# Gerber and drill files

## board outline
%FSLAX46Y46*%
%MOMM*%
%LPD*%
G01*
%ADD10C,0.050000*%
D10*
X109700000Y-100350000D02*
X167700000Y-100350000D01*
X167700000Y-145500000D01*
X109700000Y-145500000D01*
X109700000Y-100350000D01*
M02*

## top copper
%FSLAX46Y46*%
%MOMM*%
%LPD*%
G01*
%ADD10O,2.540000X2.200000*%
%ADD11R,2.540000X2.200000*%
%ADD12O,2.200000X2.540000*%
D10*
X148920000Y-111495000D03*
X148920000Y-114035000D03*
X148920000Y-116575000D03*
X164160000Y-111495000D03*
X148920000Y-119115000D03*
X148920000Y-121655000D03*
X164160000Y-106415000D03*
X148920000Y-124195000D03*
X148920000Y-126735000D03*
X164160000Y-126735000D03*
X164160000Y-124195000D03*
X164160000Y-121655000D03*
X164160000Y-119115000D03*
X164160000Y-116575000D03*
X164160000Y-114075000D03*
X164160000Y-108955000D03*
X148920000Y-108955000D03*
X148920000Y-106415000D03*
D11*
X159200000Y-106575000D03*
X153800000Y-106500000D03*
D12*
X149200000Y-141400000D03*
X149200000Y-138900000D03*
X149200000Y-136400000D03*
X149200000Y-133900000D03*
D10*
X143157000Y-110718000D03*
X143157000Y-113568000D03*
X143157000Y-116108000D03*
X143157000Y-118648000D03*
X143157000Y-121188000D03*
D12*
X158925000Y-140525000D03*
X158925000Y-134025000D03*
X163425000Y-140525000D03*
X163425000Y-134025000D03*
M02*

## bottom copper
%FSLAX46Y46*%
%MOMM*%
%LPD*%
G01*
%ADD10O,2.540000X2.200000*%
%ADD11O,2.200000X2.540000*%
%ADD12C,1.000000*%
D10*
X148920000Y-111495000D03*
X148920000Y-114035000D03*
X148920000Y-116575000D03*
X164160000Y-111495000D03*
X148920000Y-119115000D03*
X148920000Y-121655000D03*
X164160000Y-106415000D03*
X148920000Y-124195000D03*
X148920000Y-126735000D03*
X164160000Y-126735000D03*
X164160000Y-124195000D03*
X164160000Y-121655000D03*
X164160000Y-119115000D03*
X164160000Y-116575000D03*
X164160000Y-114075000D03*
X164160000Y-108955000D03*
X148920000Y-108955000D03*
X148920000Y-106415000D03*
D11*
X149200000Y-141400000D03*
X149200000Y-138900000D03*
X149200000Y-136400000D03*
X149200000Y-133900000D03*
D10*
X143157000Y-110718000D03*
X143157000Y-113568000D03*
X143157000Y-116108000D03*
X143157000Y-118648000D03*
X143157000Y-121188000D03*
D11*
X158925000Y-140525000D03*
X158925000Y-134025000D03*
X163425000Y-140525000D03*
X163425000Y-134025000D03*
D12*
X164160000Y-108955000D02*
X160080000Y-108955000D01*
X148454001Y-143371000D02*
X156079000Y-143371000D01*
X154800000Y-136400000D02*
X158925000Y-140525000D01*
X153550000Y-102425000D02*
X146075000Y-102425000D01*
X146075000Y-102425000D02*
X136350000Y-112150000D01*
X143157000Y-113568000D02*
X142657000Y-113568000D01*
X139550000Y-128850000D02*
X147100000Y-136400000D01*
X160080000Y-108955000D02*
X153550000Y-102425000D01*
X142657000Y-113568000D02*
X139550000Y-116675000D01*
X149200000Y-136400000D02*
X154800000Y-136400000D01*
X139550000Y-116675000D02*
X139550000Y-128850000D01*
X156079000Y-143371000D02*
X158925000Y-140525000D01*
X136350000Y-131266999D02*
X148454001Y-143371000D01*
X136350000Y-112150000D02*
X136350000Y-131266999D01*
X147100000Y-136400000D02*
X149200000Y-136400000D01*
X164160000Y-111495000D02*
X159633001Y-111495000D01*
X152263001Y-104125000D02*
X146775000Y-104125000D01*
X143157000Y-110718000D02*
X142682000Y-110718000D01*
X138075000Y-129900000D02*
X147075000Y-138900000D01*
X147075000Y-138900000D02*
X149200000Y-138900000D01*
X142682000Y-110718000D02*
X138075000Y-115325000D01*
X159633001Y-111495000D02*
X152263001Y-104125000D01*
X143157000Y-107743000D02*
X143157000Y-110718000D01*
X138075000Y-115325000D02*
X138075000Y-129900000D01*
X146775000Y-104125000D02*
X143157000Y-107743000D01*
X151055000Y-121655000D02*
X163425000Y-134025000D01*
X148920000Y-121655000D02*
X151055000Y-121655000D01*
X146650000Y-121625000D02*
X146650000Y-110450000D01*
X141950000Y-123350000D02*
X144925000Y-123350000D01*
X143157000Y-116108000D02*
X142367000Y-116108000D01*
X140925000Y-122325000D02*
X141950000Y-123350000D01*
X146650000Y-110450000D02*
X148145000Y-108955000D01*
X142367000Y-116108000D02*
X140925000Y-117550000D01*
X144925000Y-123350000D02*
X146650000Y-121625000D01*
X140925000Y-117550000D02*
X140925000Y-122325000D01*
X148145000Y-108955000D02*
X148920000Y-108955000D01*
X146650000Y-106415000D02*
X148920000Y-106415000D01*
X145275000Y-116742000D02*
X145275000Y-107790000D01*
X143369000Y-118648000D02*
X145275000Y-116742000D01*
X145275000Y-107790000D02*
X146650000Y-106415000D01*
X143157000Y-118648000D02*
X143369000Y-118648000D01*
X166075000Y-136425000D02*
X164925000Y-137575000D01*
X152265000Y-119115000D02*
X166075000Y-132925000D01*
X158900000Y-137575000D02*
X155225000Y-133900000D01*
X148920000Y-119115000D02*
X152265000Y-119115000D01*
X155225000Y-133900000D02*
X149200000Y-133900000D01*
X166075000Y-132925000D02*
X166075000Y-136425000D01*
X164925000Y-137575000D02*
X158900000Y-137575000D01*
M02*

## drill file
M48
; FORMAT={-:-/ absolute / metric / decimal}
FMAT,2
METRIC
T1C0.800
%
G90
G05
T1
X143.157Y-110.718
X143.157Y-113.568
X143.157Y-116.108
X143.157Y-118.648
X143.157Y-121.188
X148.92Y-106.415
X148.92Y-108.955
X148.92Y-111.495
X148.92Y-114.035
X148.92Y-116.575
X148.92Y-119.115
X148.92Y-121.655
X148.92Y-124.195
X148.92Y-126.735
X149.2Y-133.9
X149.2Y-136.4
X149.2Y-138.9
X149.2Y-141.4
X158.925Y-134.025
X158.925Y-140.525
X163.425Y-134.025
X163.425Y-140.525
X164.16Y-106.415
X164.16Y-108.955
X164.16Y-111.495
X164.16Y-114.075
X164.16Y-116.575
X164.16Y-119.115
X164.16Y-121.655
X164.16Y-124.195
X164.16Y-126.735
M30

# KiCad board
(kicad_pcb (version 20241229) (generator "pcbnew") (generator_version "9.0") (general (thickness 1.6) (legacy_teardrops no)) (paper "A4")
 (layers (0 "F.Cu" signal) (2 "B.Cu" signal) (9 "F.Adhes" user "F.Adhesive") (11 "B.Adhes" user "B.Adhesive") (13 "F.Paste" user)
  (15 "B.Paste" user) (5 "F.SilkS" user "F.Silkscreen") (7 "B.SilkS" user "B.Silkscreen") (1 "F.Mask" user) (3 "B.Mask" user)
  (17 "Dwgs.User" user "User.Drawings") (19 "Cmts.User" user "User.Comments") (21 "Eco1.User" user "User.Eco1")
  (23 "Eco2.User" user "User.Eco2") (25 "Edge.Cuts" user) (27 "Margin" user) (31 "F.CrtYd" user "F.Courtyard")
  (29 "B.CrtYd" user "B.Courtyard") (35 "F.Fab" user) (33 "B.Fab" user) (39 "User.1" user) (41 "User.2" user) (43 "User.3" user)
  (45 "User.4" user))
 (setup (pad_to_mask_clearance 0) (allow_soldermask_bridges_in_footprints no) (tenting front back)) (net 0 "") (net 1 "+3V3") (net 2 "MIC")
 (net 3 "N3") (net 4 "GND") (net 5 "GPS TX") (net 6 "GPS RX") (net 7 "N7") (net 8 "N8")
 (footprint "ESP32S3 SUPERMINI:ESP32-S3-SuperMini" (layer "F.Cu") (at 156.54 116.575)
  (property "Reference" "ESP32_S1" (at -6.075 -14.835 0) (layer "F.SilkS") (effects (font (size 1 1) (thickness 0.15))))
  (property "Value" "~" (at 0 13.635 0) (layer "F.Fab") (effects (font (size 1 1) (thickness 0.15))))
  (pad "1" thru_hole oval (at -7.62 -5.08) (size 2.54 2.2) (drill 0.8) (layers "*.Cu" "*.Mask") (remove_unused_layers no)
   (thermal_bridge_angle 45))
  (pad "2" thru_hole oval (at -7.62 -2.54) (size 2.54 2.2) (drill 0.8) (layers "*.Cu" "*.Mask") (remove_unused_layers no)
   (thermal_bridge_angle 45))
  (pad "3" thru_hole oval (at -7.62 0) (size 2.54 2.2) (drill 0.8) (layers "*.Cu" "*.Mask") (remove_unused_layers no)
   (thermal_bridge_angle 45))
  (pad "3V3" thru_hole oval (at 7.62 -5.08) (size 2.54 2.2) (drill 0.8) (layers "*.Cu" "*.Mask") (remove_unused_layers no) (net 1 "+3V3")
   (thermal_bridge_angle 45))
  (pad "4" thru_hole oval (at -7.62 2.54) (size 2.54 2.2) (drill 0.8) (layers "*.Cu" "*.Mask") (remove_unused_layers no) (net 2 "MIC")
   (thermal_bridge_angle 45))
  (pad "5" thru_hole oval (at -7.62 5.08) (size 2.54 2.2) (drill 0.8) (layers "*.Cu" "*.Mask") (remove_unused_layers no) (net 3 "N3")
   (thermal_bridge_angle 45))
  (pad "5V" thru_hole oval (at 7.62 -10.16) (size 2.54 2.2) (drill 0.8) (layers "*.Cu" "*.Mask") (remove_unused_layers no)
   (thermal_bridge_angle 45))
  (pad "6" thru_hole oval (at -7.62 7.62) (size 2.54 2.2) (drill 0.8) (layers "*.Cu" "*.Mask") (remove_unused_layers no)
   (thermal_bridge_angle 45))
  (pad "7" thru_hole oval (at -7.62 10.16) (size 2.54 2.2) (drill 0.8) (layers "*.Cu" "*.Mask") (remove_unused_layers no)
   (thermal_bridge_angle 45))
  (pad "8" thru_hole oval (at 7.62 10.16) (size 2.54 2.2) (drill 0.8) (layers "*.Cu" "*.Mask") (remove_unused_layers no)
   (thermal_bridge_angle 45))
  (pad "9" thru_hole oval (at 7.62 7.62) (size 2.54 2.2) (drill 0.8) (layers "*.Cu" "*.Mask") (remove_unused_layers no)
   (thermal_bridge_angle 45))
  (pad "10" thru_hole oval (at 7.62 5.08) (size 2.54 2.2) (drill 0.8) (layers "*.Cu" "*.Mask") (remove_unused_layers no)
   (thermal_bridge_angle 45))
  (pad "11" thru_hole oval (at 7.62 2.54) (size 2.54 2.2) (drill 0.8) (layers "*.Cu" "*.Mask") (remove_unused_layers no)
   (thermal_bridge_angle 45))
  (pad "12" thru_hole oval (at 7.62 0) (size 2.54 2.2) (drill 0.8) (layers "*.Cu" "*.Mask") (remove_unused_layers no)
   (thermal_bridge_angle 45))
  (pad "13" thru_hole oval (at 7.62 -2.5) (size 2.54 2.2) (drill 0.8) (layers "*.Cu" "*.Mask") (remove_unused_layers no)
   (thermal_bridge_angle 45))
  (pad "GND" thru_hole oval (at 7.62 -7.62) (size 2.54 2.2) (drill 0.8) (layers "*.Cu" "*.Mask") (remove_unused_layers no) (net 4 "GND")
   (thermal_bridge_angle 45))
  (pad "RX" thru_hole oval (at -7.62 -7.62) (size 2.54 2.2) (drill 0.8) (layers "*.Cu" "*.Mask") (remove_unused_layers no) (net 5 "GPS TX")
   (thermal_bridge_angle 45))
  (pad "TX" thru_hole oval (at -7.62 -10.16) (size 2.54 2.2) (drill 0.8) (layers "*.Cu" "*.Mask") (remove_unused_layers no) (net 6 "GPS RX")
   (thermal_bridge_angle 45)))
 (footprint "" (layer "F.Cu") (at 159.2 106.575)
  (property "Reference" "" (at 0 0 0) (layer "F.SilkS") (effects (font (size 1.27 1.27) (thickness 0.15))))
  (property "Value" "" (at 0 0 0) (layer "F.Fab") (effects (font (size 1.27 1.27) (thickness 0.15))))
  (pad "3V3" smd rect (at 0 0) (size 2.54 2.2) (layers "F.Cu" "F.Mask" "F.Paste") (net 1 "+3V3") (thermal_bridge_angle 45)))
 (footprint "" (layer "F.Cu") (at 153.8 106.5)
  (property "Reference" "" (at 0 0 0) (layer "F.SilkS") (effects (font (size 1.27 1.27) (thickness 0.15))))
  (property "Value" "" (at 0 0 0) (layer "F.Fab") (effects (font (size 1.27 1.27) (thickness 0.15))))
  (pad "GND" smd rect (at 0 0) (size 2.54 2.2) (layers "F.Cu" "F.Mask" "F.Paste") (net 4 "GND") (thermal_bridge_angle 45)))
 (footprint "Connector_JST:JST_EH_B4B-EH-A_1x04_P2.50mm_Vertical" (layer "F.Cu") (at 149.2 141.4 90)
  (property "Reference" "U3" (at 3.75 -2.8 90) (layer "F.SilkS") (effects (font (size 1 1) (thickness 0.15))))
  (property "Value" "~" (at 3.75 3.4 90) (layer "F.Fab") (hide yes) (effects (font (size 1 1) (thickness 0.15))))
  (pad "1" thru_hole oval (at 0 0 90) (size 2.54 2.2) (drill 0.8) (layers "*.Cu" "*.Mask") (remove_unused_layers no) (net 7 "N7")
   (thermal_bridge_angle 45))
  (pad "2" thru_hole oval (at 2.5 0 90) (size 2.54 2.2) (drill 0.8) (layers "*.Cu" "*.Mask") (remove_unused_layers no) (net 1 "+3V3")
   (thermal_bridge_angle 45))
  (pad "3" thru_hole oval (at 5 0 90) (size 2.54 2.2) (drill 0.8) (layers "*.Cu" "*.Mask") (remove_unused_layers no) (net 4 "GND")
   (thermal_bridge_angle 45))
  (pad "4" thru_hole oval (at 7.5 0 90) (size 2.54 2.2) (drill 0.8) (layers "*.Cu" "*.Mask") (remove_unused_layers no) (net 2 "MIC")
   (thermal_bridge_angle 45)))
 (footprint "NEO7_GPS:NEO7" (layer "F.Cu") (at 92.738 102.9)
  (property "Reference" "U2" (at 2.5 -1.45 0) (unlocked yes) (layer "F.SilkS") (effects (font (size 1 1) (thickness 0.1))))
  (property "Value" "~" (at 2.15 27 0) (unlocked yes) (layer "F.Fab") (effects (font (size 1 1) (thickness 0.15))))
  (pad "1" thru_hole oval (at 50.419 7.818) (size 2.54 2.2) (drill 0.8) (layers "*.Cu" "*.Mask") (remove_unused_layers no) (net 1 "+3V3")
   (thermal_bridge_angle 45))
  (pad "2" thru_hole oval (at 50.419 10.668) (size 2.54 2.2) (drill 0.8) (layers "*.Cu" "*.Mask") (remove_unused_layers no) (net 4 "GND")
   (thermal_bridge_angle 45))
  (pad "3" thru_hole oval (at 50.419 13.208) (size 2.54 2.2) (drill 0.8) (layers "*.Cu" "*.Mask") (remove_unused_layers no) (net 5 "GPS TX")
   (thermal_bridge_angle 45))
  (pad "4" thru_hole oval (at 50.419 15.748) (size 2.54 2.2) (drill 0.8) (layers "*.Cu" "*.Mask") (remove_unused_layers no) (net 6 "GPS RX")
   (thermal_bridge_angle 45))
  (pad "5" thru_hole oval (at 50.419 18.288) (size 2.54 2.2) (drill 0.8) (layers "*.Cu" "*.Mask") (remove_unused_layers no) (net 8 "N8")
   (thermal_bridge_angle 45)))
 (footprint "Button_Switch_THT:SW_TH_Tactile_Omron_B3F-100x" (layer "F.Cu") (at 158.925 140.525 90)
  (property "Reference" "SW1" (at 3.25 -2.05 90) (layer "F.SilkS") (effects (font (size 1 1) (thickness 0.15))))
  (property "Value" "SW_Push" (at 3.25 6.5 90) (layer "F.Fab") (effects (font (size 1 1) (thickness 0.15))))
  (pad "1" thru_hole oval (at 0 0 90) (size 2.54 2.2) (drill 0.8) (layers "*.Cu" "*.Mask") (remove_unused_layers no) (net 4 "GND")
   (thermal_bridge_angle 45))
  (pad "1" thru_hole oval (at 6.5 0 90) (size 2.54 2.2) (drill 0.8) (layers "*.Cu" "*.Mask") (remove_unused_layers no) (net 4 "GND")
   (thermal_bridge_angle 45))
  (pad "2" thru_hole oval (at 0 4.5 90) (size 2.54 2.2) (drill 0.8) (layers "*.Cu" "*.Mask") (remove_unused_layers no) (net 3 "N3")
   (thermal_bridge_angle 45))
  (pad "2" thru_hole oval (at 6.5 4.5 90) (size 2.54 2.2) (drill 0.8) (layers "*.Cu" "*.Mask") (remove_unused_layers no) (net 3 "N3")
   (thermal_bridge_angle 45)))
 (gr_rect (start 109.7 100.35) (end 167.7 145.5) (stroke (width 0.05) (type solid)) (fill no) (layer "Edge.Cuts"))
 (segment (start 164.16 108.955) (end 160.08 108.955) (width 1) (layer "B.Cu") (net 4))
 (segment (start 148.454001 143.371) (end 156.079 143.371) (width 1) (layer "B.Cu") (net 4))
 (segment (start 154.8 136.4) (end 158.925 140.525) (width 1) (layer "B.Cu") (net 4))
 (segment (start 153.55 102.425) (end 146.075 102.425) (width 1) (layer "B.Cu") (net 4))
 (segment (start 146.075 102.425) (end 136.35 112.15) (width 1) (layer "B.Cu") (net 4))
 (segment (start 143.157 113.568) (end 142.657 113.568) (width 1) (layer "B.Cu") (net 4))
 (segment (start 139.55 128.85) (end 147.1 136.4) (width 1) (layer "B.Cu") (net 4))
 (segment (start 160.08 108.955) (end 153.55 102.425) (width 1) (layer "B.Cu") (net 4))
 (segment (start 142.657 113.568) (end 139.55 116.675) (width 1) (layer "B.Cu") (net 4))
 (segment (start 149.2 136.4) (end 154.8 136.4) (width 1) (layer "B.Cu") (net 4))
 (segment (start 139.55 116.675) (end 139.55 128.85) (width 1) (layer "B.Cu") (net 4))
 (segment (start 156.079 143.371) (end 158.925 140.525) (width 1) (layer "B.Cu") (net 4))
 (segment (start 136.35 131.266999) (end 148.454001 143.371) (width 1) (layer "B.Cu") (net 4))
 (segment (start 136.35 112.15) (end 136.35 131.266999) (width 1) (layer "B.Cu") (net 4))
 (segment (start 147.1 136.4) (end 149.2 136.4) (width 1) (layer "B.Cu") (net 4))
 (segment (start 164.16 111.495) (end 159.633001 111.495) (width 1) (layer "B.Cu") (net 1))
 (segment (start 152.263001 104.125) (end 146.775 104.125) (width 1) (layer "B.Cu") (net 1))
 (segment (start 143.157 110.718) (end 142.682 110.718) (width 1) (layer "B.Cu") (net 1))
 (segment (start 138.075 129.9) (end 147.075 138.9) (width 1) (layer "B.Cu") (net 1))
 (segment (start 147.075 138.9) (end 149.2 138.9) (width 1) (layer "B.Cu") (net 1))
 (segment (start 142.682 110.718) (end 138.075 115.325) (width 1) (layer "B.Cu") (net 1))
 (segment (start 159.633001 111.495) (end 152.263001 104.125) (width 1) (layer "B.Cu") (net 1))
 (segment (start 143.157 107.743) (end 143.157 110.718) (width 1) (layer "B.Cu") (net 1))
 (segment (start 138.075 115.325) (end 138.075 129.9) (width 1) (layer "B.Cu") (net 1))
 (segment (start 146.775 104.125) (end 143.157 107.743) (width 1) (layer "B.Cu") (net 1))
 (segment (start 151.055 121.655) (end 163.425 134.025) (width 1) (layer "B.Cu") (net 3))
 (segment (start 148.92 121.655) (end 151.055 121.655) (width 1) (layer "B.Cu") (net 3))
 (segment (start 146.65 121.625) (end 146.65 110.45) (width 1) (layer "B.Cu") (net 5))
 (segment (start 141.95 123.35) (end 144.925 123.35) (width 1) (layer "B.Cu") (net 5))
 (segment (start 143.157 116.108) (end 142.367 116.108) (width 1) (layer "B.Cu") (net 5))
 (segment (start 140.925 122.325) (end 141.95 123.35) (width 1) (layer "B.Cu") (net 5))
 (segment (start 146.65 110.45) (end 148.145 108.955) (width 1) (layer "B.Cu") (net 5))
 (segment (start 142.367 116.108) (end 140.925 117.55) (width 1) (layer "B.Cu") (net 5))
 (segment (start 144.925 123.35) (end 146.65 121.625) (width 1) (layer "B.Cu") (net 5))
 (segment (start 140.925 117.55) (end 140.925 122.325) (width 1) (layer "B.Cu") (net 5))
 (segment (start 148.145 108.955) (end 148.92 108.955) (width 1) (layer "B.Cu") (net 5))
 (segment (start 146.65 106.415) (end 148.92 106.415) (width 1) (layer "B.Cu") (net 6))
 (segment (start 145.275 116.742) (end 145.275 107.79) (width 1) (layer "B.Cu") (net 6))
 (segment (start 143.369 118.648) (end 145.275 116.742) (width 1) (layer "B.Cu") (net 6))
 (segment (start 145.275 107.79) (end 146.65 106.415) (width 1) (layer "B.Cu") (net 6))
 (segment (start 143.157 118.648) (end 143.369 118.648) (width 1) (layer "B.Cu") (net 6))
 (segment (start 166.075 136.425) (end 164.925 137.575) (width 1) (layer "B.Cu") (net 2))
 (segment (start 152.265 119.115) (end 166.075 132.925) (width 1) (layer "B.Cu") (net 2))
 (segment (start 158.9 137.575) (end 155.225 133.9) (width 1) (layer "B.Cu") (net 2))
 (segment (start 148.92 119.115) (end 152.265 119.115) (width 1) (layer "B.Cu") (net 2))
 (segment (start 155.225 133.9) (end 149.2 133.9) (width 1) (layer "B.Cu") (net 2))
 (segment (start 166.075 132.925) (end 166.075 136.425) (width 1) (layer "B.Cu") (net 2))
 (segment (start 164.925 137.575) (end 158.9 137.575) (width 1) (layer "B.Cu") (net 2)))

